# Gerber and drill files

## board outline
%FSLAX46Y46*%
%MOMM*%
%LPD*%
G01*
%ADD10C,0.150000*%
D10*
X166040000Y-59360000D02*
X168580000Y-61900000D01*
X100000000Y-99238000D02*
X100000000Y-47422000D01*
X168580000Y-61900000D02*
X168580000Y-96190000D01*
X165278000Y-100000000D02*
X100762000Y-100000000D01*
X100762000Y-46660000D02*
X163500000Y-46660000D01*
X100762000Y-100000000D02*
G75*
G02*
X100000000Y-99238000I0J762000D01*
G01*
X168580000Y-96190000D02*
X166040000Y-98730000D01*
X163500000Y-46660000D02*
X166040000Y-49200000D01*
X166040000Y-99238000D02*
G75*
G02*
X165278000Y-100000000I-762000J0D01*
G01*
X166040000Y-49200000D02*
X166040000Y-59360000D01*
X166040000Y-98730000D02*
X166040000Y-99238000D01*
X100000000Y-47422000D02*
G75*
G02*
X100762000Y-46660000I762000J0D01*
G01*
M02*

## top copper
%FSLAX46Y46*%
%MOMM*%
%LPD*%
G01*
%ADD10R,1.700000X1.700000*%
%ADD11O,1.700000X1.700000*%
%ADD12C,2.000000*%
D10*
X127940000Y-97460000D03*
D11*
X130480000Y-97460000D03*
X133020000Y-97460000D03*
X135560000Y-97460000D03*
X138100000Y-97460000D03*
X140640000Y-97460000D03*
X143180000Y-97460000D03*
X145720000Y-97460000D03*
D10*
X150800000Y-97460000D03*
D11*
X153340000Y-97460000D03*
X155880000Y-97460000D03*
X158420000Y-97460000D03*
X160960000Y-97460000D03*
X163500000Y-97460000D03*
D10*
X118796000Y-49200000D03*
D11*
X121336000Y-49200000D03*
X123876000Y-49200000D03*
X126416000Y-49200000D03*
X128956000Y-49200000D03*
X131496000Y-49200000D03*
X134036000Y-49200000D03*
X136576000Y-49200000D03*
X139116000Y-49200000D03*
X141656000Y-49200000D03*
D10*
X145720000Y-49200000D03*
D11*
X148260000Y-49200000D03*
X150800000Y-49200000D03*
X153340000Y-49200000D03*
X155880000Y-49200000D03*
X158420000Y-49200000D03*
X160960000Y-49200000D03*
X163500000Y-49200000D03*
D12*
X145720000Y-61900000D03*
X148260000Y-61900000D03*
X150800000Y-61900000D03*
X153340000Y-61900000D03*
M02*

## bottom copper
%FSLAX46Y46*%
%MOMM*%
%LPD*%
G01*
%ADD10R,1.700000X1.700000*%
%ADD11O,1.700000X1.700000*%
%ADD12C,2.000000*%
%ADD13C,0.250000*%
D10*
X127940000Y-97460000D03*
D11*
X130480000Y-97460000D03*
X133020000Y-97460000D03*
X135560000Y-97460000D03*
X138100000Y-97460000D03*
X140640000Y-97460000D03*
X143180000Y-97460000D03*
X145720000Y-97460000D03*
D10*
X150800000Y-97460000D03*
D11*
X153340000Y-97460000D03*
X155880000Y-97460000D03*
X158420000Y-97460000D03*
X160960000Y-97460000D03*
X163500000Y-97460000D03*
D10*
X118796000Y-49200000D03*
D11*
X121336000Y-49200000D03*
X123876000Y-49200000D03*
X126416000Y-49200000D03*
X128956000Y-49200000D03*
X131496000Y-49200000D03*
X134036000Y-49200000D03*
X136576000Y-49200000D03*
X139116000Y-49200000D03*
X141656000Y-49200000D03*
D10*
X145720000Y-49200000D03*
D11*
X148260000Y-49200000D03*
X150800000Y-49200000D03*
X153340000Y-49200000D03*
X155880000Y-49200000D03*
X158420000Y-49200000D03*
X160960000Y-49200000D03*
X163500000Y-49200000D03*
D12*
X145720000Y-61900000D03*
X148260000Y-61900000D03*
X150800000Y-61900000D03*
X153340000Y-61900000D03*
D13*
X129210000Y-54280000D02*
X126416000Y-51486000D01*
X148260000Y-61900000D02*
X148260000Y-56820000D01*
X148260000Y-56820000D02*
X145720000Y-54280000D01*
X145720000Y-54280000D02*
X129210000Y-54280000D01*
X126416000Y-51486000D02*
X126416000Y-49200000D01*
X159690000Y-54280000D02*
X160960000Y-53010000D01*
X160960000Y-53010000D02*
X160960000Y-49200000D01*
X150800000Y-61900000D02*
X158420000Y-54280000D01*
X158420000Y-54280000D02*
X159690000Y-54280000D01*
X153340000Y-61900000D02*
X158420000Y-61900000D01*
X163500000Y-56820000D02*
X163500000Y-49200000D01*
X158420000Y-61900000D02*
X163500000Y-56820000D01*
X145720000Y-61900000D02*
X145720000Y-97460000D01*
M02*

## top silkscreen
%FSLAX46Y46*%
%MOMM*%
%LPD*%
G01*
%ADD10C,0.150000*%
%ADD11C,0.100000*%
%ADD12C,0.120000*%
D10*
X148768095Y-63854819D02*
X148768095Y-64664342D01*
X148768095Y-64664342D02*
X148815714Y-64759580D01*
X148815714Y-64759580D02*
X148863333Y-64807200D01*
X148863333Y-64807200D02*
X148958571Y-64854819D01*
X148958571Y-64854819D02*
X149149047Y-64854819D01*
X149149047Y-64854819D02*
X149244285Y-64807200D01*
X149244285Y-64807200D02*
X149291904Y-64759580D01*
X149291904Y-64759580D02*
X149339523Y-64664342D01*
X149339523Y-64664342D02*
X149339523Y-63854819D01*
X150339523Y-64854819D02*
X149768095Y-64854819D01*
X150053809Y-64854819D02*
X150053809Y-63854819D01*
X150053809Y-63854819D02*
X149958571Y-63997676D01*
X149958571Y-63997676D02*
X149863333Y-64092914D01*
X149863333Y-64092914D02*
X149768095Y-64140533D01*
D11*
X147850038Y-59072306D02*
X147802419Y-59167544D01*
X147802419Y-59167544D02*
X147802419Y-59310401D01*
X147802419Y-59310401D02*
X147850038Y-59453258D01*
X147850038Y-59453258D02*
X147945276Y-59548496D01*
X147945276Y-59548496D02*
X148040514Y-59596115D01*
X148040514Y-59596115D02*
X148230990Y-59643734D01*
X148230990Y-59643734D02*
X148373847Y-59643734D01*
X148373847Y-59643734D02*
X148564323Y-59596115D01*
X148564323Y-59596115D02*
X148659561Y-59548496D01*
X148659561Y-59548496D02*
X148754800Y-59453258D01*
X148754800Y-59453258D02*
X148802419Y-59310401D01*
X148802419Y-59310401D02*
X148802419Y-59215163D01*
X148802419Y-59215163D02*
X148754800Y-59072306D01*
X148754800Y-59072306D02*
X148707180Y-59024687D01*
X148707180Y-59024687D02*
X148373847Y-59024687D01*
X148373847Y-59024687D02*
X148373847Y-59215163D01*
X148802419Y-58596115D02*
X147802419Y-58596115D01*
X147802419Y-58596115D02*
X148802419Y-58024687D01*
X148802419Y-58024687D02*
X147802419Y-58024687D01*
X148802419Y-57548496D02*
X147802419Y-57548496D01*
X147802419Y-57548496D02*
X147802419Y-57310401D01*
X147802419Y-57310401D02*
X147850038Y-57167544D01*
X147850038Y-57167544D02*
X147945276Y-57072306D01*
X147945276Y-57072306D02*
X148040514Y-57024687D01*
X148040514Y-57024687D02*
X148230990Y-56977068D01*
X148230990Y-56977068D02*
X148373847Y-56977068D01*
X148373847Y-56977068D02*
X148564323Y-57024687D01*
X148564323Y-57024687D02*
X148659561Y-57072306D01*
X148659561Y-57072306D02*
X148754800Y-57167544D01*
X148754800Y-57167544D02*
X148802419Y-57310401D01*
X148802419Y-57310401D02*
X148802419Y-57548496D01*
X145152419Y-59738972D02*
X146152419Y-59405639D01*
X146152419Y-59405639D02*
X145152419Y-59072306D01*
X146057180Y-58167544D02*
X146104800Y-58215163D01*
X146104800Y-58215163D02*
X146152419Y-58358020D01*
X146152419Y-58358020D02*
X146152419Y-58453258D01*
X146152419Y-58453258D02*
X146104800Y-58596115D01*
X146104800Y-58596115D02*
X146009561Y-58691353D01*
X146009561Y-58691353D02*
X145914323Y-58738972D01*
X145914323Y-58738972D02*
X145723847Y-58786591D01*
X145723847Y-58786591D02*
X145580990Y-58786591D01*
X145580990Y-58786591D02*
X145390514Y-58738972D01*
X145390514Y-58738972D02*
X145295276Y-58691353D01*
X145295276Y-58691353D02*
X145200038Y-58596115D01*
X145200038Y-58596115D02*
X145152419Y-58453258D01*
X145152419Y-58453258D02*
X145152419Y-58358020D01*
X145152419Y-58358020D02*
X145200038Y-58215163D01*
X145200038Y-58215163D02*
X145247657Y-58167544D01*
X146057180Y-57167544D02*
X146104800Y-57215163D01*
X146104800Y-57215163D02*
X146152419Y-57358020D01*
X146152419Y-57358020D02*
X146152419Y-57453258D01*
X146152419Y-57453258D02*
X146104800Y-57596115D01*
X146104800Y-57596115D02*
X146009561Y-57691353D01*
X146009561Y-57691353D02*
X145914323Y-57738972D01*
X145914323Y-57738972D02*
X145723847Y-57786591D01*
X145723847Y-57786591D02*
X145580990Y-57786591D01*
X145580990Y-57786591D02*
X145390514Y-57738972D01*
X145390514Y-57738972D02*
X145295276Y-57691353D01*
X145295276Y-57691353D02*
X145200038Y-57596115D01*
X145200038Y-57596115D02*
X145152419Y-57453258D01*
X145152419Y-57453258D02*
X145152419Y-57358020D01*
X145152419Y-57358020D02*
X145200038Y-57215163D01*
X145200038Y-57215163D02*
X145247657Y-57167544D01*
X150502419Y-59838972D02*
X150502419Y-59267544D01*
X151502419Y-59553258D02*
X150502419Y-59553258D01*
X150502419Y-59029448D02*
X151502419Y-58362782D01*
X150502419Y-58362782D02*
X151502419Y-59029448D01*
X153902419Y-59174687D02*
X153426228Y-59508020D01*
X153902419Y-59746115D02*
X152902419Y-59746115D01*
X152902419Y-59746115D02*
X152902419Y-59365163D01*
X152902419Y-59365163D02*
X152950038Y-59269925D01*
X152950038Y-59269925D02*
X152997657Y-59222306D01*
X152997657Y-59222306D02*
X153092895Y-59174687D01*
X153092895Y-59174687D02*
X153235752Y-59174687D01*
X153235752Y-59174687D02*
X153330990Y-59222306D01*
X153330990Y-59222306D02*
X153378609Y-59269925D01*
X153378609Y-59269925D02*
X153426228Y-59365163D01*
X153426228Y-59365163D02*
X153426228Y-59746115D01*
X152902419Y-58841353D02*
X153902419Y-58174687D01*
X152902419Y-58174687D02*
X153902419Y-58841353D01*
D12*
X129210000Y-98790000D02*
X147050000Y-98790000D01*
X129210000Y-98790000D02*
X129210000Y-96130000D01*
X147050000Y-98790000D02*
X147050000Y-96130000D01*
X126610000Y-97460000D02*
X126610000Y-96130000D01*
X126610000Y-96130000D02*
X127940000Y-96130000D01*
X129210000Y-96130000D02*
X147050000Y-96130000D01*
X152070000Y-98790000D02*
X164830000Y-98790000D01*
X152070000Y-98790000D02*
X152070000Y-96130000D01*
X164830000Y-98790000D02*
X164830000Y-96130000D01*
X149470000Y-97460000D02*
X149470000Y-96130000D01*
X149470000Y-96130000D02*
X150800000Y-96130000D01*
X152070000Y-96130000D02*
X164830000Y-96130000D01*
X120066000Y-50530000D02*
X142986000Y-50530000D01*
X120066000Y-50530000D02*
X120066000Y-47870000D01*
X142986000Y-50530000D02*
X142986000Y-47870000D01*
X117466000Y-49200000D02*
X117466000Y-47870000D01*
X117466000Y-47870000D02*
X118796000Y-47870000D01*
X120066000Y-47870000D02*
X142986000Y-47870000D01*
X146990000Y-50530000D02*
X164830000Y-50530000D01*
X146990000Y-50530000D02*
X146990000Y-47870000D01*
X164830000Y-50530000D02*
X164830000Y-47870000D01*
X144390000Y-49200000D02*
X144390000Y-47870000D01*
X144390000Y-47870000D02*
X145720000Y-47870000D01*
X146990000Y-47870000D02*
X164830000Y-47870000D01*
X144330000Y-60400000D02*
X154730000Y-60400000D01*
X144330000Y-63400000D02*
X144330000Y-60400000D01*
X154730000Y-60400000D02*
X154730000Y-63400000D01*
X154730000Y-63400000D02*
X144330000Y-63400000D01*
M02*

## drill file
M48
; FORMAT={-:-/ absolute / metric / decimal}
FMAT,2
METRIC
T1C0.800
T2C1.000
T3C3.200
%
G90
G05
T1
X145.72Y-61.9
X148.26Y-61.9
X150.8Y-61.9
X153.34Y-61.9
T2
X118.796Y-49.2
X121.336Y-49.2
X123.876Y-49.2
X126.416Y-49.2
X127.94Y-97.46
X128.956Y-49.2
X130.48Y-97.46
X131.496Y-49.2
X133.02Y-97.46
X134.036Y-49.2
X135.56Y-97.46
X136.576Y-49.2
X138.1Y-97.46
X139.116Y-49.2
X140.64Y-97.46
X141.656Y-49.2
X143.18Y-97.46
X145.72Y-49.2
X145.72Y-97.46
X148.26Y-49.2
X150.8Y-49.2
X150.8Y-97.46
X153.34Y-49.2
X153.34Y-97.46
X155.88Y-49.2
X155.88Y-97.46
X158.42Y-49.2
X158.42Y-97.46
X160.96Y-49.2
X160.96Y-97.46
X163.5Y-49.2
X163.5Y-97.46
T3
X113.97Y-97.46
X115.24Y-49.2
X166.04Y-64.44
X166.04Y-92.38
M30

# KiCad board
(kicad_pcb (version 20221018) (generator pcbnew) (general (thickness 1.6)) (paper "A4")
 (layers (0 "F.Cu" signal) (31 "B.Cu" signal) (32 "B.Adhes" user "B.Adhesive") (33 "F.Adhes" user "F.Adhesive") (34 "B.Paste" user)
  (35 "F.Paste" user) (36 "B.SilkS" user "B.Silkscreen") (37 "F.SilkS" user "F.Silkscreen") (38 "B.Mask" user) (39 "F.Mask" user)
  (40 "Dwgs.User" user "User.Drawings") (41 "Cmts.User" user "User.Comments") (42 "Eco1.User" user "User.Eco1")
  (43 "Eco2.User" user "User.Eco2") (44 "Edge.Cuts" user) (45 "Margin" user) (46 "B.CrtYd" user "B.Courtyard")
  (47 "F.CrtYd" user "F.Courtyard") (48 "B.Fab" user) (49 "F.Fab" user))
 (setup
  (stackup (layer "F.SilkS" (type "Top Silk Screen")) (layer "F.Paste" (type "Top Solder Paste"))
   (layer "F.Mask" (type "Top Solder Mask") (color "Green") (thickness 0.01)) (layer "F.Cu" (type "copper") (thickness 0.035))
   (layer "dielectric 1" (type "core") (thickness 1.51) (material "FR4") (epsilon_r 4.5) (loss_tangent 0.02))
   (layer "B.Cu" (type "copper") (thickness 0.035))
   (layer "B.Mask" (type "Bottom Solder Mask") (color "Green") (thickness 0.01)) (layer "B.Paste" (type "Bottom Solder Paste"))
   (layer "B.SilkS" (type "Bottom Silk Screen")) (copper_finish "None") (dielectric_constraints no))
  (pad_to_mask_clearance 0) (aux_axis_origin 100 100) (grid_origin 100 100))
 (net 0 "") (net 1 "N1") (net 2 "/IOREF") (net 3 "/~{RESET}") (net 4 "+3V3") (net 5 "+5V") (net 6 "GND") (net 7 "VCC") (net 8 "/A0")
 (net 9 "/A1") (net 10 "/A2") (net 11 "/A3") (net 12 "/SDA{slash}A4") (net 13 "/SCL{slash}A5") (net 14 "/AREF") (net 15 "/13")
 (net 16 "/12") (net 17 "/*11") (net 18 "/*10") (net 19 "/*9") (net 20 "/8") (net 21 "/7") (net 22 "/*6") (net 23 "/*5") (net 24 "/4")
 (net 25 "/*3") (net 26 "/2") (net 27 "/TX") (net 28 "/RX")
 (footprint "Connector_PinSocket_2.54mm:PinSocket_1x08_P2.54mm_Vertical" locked (layer "F.Cu") (at 127.94 97.46 90)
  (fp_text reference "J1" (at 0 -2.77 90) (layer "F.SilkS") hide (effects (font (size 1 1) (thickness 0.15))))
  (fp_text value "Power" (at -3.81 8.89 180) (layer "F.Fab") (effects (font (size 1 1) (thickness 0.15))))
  (fp_line (start -1.33 1.27) (end -1.33 19.11) (stroke (width 0.12) (type solid)) (layer "F.SilkS"))
  (fp_line (start -1.33 1.27) (end 1.33 1.27) (stroke (width 0.12) (type solid)) (layer "F.SilkS"))
  (fp_line (start -1.33 19.11) (end 1.33 19.11) (stroke (width 0.12) (type solid)) (layer "F.SilkS"))
  (fp_line (start 0 -1.33) (end 1.33 -1.33) (stroke (width 0.12) (type solid)) (layer "F.SilkS"))
  (fp_line (start 1.33 -1.33) (end 1.33 0) (stroke (width 0.12) (type solid)) (layer "F.SilkS"))
  (fp_line (start 1.33 1.27) (end 1.33 19.11) (stroke (width 0.12) (type solid)) (layer "F.SilkS"))
  (pad "1" thru_hole rect locked (at 0 0 90) (size 1.7 1.7) (drill 1) (layers "*.Cu" "*.Mask") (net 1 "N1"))
  (pad "2" thru_hole oval locked (at 0 2.54 90) (size 1.7 1.7) (drill 1) (layers "*.Cu" "*.Mask") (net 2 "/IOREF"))
  (pad "3" thru_hole oval locked (at 0 5.08 90) (size 1.7 1.7) (drill 1) (layers "*.Cu" "*.Mask") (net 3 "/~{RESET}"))
  (pad "4" thru_hole oval locked (at 0 7.62 90) (size 1.7 1.7) (drill 1) (layers "*.Cu" "*.Mask") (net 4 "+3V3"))
  (pad "5" thru_hole oval locked (at 0 10.16 90) (size 1.7 1.7) (drill 1) (layers "*.Cu" "*.Mask") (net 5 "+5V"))
  (pad "6" thru_hole oval locked (at 0 12.7 90) (size 1.7 1.7) (drill 1) (layers "*.Cu" "*.Mask") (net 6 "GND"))
  (pad "7" thru_hole oval locked (at 0 15.24 90) (size 1.7 1.7) (drill 1) (layers "*.Cu" "*.Mask") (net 6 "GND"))
  (pad "8" thru_hole oval locked (at 0 17.78 90) (size 1.7 1.7) (drill 1) (layers "*.Cu" "*.Mask") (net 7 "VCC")))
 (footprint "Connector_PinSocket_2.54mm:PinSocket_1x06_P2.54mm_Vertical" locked (layer "F.Cu") (at 150.8 97.46 90)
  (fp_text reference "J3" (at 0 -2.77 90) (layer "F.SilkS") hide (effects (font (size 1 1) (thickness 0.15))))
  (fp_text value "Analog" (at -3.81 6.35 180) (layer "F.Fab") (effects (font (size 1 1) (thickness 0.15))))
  (fp_line (start -1.33 1.27) (end -1.33 14.03) (stroke (width 0.12) (type solid)) (layer "F.SilkS"))
  (fp_line (start -1.33 1.27) (end 1.33 1.27) (stroke (width 0.12) (type solid)) (layer "F.SilkS"))
  (fp_line (start -1.33 14.03) (end 1.33 14.03) (stroke (width 0.12) (type solid)) (layer "F.SilkS"))
  (fp_line (start 0 -1.33) (end 1.33 -1.33) (stroke (width 0.12) (type solid)) (layer "F.SilkS"))
  (fp_line (start 1.33 -1.33) (end 1.33 0) (stroke (width 0.12) (type solid)) (layer "F.SilkS"))
  (fp_line (start 1.33 1.27) (end 1.33 14.03) (stroke (width 0.12) (type solid)) (layer "F.SilkS"))
  (pad "1" thru_hole rect locked (at 0 0 90) (size 1.7 1.7) (drill 1) (layers "*.Cu" "*.Mask") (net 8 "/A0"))
  (pad "2" thru_hole oval locked (at 0 2.54 90) (size 1.7 1.7) (drill 1) (layers "*.Cu" "*.Mask") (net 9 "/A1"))
  (pad "3" thru_hole oval locked (at 0 5.08 90) (size 1.7 1.7) (drill 1) (layers "*.Cu" "*.Mask") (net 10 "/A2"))
  (pad "4" thru_hole oval locked (at 0 7.62 90) (size 1.7 1.7) (drill 1) (layers "*.Cu" "*.Mask") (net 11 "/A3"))
  (pad "5" thru_hole oval locked (at 0 10.16 90) (size 1.7 1.7) (drill 1) (layers "*.Cu" "*.Mask") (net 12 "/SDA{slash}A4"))
  (pad "6" thru_hole oval locked (at 0 12.7 90) (size 1.7 1.7) (drill 1) (layers "*.Cu" "*.Mask") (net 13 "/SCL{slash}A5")))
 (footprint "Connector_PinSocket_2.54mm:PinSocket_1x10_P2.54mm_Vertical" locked (layer "F.Cu") (at 118.796 49.2 90)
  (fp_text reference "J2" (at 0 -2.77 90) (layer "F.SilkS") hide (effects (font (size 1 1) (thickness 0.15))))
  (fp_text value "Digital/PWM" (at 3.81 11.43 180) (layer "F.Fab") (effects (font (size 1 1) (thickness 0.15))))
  (fp_line (start -1.33 1.27) (end -1.33 24.19) (stroke (width 0.12) (type solid)) (layer "F.SilkS"))
  (fp_line (start -1.33 1.27) (end 1.33 1.27) (stroke (width 0.12) (type solid)) (layer "F.SilkS"))
  (fp_line (start -1.33 24.19) (end 1.33 24.19) (stroke (width 0.12) (type solid)) (layer "F.SilkS"))
  (fp_line (start 0 -1.33) (end 1.33 -1.33) (stroke (width 0.12) (type solid)) (layer "F.SilkS"))
  (fp_line (start 1.33 -1.33) (end 1.33 0) (stroke (width 0.12) (type solid)) (layer "F.SilkS"))
  (fp_line (start 1.33 1.27) (end 1.33 24.19) (stroke (width 0.12) (type solid)) (layer "F.SilkS"))
  (pad "1" thru_hole rect locked (at 0 0 90) (size 1.7 1.7) (drill 1) (layers "*.Cu" "*.Mask") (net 13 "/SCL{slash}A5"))
  (pad "2" thru_hole oval locked (at 0 2.54 90) (size 1.7 1.7) (drill 1) (layers "*.Cu" "*.Mask") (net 12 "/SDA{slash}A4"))
  (pad "3" thru_hole oval locked (at 0 5.08 90) (size 1.7 1.7) (drill 1) (layers "*.Cu" "*.Mask") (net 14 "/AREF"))
  (pad "4" thru_hole oval locked (at 0 7.62 90) (size 1.7 1.7) (drill 1) (layers "*.Cu" "*.Mask") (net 6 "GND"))
  (pad "5" thru_hole oval locked (at 0 10.16 90) (size 1.7 1.7) (drill 1) (layers "*.Cu" "*.Mask") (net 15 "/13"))
  (pad "6" thru_hole oval locked (at 0 12.7 90) (size 1.7 1.7) (drill 1) (layers "*.Cu" "*.Mask") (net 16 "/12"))
  (pad "7" thru_hole oval locked (at 0 15.24 90) (size 1.7 1.7) (drill 1) (layers "*.Cu" "*.Mask") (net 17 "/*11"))
  (pad "8" thru_hole oval locked (at 0 17.78 90) (size 1.7 1.7) (drill 1) (layers "*.Cu" "*.Mask") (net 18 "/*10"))
  (pad "9" thru_hole oval locked (at 0 20.32 90) (size 1.7 1.7) (drill 1) (layers "*.Cu" "*.Mask") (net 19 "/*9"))
  (pad "10" thru_hole oval locked (at 0 22.86 90) (size 1.7 1.7) (drill 1) (layers "*.Cu" "*.Mask") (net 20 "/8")))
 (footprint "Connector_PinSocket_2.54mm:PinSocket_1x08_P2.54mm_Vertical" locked (layer "F.Cu") (at 145.72 49.2 90)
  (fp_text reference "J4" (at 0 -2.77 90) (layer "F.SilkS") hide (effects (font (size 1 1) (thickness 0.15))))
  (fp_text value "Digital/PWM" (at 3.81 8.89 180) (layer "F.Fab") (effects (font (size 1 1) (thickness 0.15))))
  (fp_line (start -1.33 1.27) (end -1.33 19.11) (stroke (width 0.12) (type solid)) (layer "F.SilkS"))
  (fp_line (start -1.33 1.27) (end 1.33 1.27) (stroke (width 0.12) (type solid)) (layer "F.SilkS"))
  (fp_line (start -1.33 19.11) (end 1.33 19.11) (stroke (width 0.12) (type solid)) (layer "F.SilkS"))
  (fp_line (start 0 -1.33) (end 1.33 -1.33) (stroke (width 0.12) (type solid)) (layer "F.SilkS"))
  (fp_line (start 1.33 -1.33) (end 1.33 0) (stroke (width 0.12) (type solid)) (layer "F.SilkS"))
  (fp_line (start 1.33 1.27) (end 1.33 19.11) (stroke (width 0.12) (type solid)) (layer "F.SilkS"))
  (pad "1" thru_hole rect locked (at 0 0 90) (size 1.7 1.7) (drill 1) (layers "*.Cu" "*.Mask") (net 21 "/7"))
  (pad "2" thru_hole oval locked (at 0 2.54 90) (size 1.7 1.7) (drill 1) (layers "*.Cu" "*.Mask") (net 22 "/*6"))
  (pad "3" thru_hole oval locked (at 0 5.08 90) (size 1.7 1.7) (drill 1) (layers "*.Cu" "*.Mask") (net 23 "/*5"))
  (pad "4" thru_hole oval locked (at 0 7.62 90) (size 1.7 1.7) (drill 1) (layers "*.Cu" "*.Mask") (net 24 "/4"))
  (pad "5" thru_hole oval locked (at 0 10.16 90) (size 1.7 1.7) (drill 1) (layers "*.Cu" "*.Mask") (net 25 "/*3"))
  (pad "6" thru_hole oval locked (at 0 12.7 90) (size 1.7 1.7) (drill 1) (layers "*.Cu" "*.Mask") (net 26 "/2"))
  (pad "7" thru_hole oval locked (at 0 15.24 90) (size 1.7 1.7) (drill 1) (layers "*.Cu" "*.Mask") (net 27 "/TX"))
  (pad "8" thru_hole oval locked (at 0 17.78 90) (size 1.7 1.7) (drill 1) (layers "*.Cu" "*.Mask") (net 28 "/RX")))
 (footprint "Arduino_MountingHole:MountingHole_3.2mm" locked (layer "F.Cu") (at 115.24 49.2)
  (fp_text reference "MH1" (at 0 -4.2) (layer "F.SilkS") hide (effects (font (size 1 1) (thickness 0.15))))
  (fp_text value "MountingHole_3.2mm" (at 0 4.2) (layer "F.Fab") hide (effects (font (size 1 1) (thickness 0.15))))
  (pad "" np_thru_hole circle locked (at 0 0) (size 3.2 3.2) (drill 3.2) (layers "*.Cu" "*.Mask")))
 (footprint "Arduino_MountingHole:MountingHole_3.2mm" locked (layer "F.Cu") (at 113.97 97.46)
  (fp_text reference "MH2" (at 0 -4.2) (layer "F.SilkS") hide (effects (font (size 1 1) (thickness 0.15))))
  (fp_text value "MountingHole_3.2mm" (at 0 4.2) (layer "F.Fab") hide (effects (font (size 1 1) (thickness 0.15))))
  (pad "" np_thru_hole circle locked (at 0 0) (size 3.2 3.2) (drill 3.2) (layers "*.Cu" "*.Mask")))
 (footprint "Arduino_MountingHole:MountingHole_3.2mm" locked (layer "F.Cu") (at 166.04 64.44)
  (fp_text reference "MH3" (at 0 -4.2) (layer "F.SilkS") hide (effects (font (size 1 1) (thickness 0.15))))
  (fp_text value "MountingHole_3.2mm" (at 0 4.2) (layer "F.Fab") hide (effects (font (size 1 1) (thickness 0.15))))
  (pad "" np_thru_hole circle locked (at 0 0) (size 3.2 3.2) (drill 3.2) (layers "*.Cu" "*.Mask")))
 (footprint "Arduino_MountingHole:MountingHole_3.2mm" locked (layer "F.Cu") (at 166.04 92.38)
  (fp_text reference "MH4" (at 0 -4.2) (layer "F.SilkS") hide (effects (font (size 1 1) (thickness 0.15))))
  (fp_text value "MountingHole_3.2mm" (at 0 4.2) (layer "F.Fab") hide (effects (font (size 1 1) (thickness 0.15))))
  (pad "" np_thru_hole circle locked (at 0 0) (size 3.2 3.2) (drill 3.2) (layers "*.Cu" "*.Mask")))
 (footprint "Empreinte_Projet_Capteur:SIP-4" (layer "F.Cu") (at 149.53 61.9)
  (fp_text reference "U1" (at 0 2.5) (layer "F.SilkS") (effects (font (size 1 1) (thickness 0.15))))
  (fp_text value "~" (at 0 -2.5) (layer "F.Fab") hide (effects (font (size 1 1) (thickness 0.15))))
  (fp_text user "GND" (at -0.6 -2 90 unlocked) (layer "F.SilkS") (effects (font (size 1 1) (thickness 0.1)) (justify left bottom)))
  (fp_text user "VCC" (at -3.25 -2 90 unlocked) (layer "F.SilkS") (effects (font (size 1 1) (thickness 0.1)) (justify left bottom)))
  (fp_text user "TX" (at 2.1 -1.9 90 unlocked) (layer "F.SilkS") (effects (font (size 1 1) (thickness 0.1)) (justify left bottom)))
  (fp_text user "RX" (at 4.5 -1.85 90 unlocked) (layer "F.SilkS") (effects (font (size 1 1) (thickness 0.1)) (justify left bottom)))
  (fp_line (start -5.2 -1.5) (end 5.2 -1.5) (stroke (width 0.12) (type default)) (layer "F.SilkS"))
  (fp_line (start -5.2 1.5) (end -5.2 -1.5) (stroke (width 0.12) (type default)) (layer "F.SilkS"))
  (fp_line (start 5.2 -1.5) (end 5.2 1.5) (stroke (width 0.12) (type default)) (layer "F.SilkS"))
  (fp_line (start 5.2 1.5) (end -5.2 1.5) (stroke (width 0.12) (type default)) (layer "F.SilkS"))
  (pad "1" thru_hole circle (at -3.81 0) (size 2 2) (drill 0.8) (layers "*.Cu" "*.Mask") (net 7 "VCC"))
  (pad "2" thru_hole circle (at -1.27 0) (size 2 2) (drill 0.8) (layers "*.Cu" "*.Mask") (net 6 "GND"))
  (pad "3" thru_hole circle (at 1.27 0) (size 2 2) (drill 0.8) (layers "*.Cu" "*.Mask") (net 27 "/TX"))
  (pad "4" thru_hole circle (at 3.81 0) (size 2 2) (drill 0.8) (layers "*.Cu" "*.Mask") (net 28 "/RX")))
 (gr_line (start 166.04 59.36) (end 168.58 61.9) (stroke (width 0.15) (type solid)) (layer "Edge.Cuts"))
 (gr_line (start 100 99.238) (end 100 47.422) (stroke (width 0.15) (type solid)) (layer "Edge.Cuts"))
 (gr_line (start 168.58 61.9) (end 168.58 96.19) (stroke (width 0.15) (type solid)) (layer "Edge.Cuts"))
 (gr_line (start 165.278 100) (end 100.762 100) (stroke (width 0.15) (type solid)) (layer "Edge.Cuts"))
 (gr_line (start 100.762 46.66) (end 163.5 46.66) (stroke (width 0.15) (type solid)) (layer "Edge.Cuts"))
 (gr_arc (start 100.762 100) (mid 100.223185 99.776815) (end 100 99.238) (stroke (width 0.15) (type solid)) (layer "Edge.Cuts"))
 (gr_line (start 168.58 96.19) (end 166.04 98.73) (stroke (width 0.15) (type solid)) (layer "Edge.Cuts"))
 (gr_line (start 163.5 46.66) (end 166.04 49.2) (stroke (width 0.15) (type solid)) (layer "Edge.Cuts"))
 (gr_arc (start 166.04 99.238) (mid 165.816815 99.776815) (end 165.278 100) (stroke (width 0.15) (type solid)) (layer "Edge.Cuts"))
 (gr_line (start 166.04 49.2) (end 166.04 59.36) (stroke (width 0.15) (type solid)) (layer "Edge.Cuts"))
 (gr_line (start 166.04 98.73) (end 166.04 99.238) (stroke (width 0.15) (type solid)) (layer "Edge.Cuts"))
 (gr_arc (start 100 47.422) (mid 100.223185 46.883185) (end 100.762 46.66) (stroke (width 0.15) (type solid)) (layer "Edge.Cuts"))
 (segment (start 129.21 54.28) (end 126.416 51.486) (width 0.25) (layer "B.Cu") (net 6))
 (segment (start 148.26 61.9) (end 148.26 56.82) (width 0.25) (layer "B.Cu") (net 6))
 (segment (start 148.26 56.82) (end 145.72 54.28) (width 0.25) (layer "B.Cu") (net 6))
 (segment (start 145.72 54.28) (end 129.21 54.28) (width 0.25) (layer "B.Cu") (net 6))
 (segment (start 126.416 51.486) (end 126.416 49.2) (width 0.25) (layer "B.Cu") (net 6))
 (segment (start 159.69 54.28) (end 160.96 53.01) (width 0.25) (layer "B.Cu") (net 27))
 (segment (start 160.96 53.01) (end 160.96 49.2) (width 0.25) (layer "B.Cu") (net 27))
 (segment (start 150.8 61.9) (end 158.42 54.28) (width 0.25) (layer "B.Cu") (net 27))
 (segment (start 158.42 54.28) (end 159.69 54.28) (width 0.25) (layer "B.Cu") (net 27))
 (segment (start 153.34 61.9) (end 158.42 61.9) (width 0.25) (layer "B.Cu") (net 28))
 (segment (start 163.5 56.82) (end 163.5 49.2) (width 0.25) (layer "B.Cu") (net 28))
 (segment (start 158.42 61.9) (end 163.5 56.82) (width 0.25) (layer "B.Cu") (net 28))
 (segment (start 145.72 61.9) (end 145.72 97.46) (width 0.25) (layer "B.Cu") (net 7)))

